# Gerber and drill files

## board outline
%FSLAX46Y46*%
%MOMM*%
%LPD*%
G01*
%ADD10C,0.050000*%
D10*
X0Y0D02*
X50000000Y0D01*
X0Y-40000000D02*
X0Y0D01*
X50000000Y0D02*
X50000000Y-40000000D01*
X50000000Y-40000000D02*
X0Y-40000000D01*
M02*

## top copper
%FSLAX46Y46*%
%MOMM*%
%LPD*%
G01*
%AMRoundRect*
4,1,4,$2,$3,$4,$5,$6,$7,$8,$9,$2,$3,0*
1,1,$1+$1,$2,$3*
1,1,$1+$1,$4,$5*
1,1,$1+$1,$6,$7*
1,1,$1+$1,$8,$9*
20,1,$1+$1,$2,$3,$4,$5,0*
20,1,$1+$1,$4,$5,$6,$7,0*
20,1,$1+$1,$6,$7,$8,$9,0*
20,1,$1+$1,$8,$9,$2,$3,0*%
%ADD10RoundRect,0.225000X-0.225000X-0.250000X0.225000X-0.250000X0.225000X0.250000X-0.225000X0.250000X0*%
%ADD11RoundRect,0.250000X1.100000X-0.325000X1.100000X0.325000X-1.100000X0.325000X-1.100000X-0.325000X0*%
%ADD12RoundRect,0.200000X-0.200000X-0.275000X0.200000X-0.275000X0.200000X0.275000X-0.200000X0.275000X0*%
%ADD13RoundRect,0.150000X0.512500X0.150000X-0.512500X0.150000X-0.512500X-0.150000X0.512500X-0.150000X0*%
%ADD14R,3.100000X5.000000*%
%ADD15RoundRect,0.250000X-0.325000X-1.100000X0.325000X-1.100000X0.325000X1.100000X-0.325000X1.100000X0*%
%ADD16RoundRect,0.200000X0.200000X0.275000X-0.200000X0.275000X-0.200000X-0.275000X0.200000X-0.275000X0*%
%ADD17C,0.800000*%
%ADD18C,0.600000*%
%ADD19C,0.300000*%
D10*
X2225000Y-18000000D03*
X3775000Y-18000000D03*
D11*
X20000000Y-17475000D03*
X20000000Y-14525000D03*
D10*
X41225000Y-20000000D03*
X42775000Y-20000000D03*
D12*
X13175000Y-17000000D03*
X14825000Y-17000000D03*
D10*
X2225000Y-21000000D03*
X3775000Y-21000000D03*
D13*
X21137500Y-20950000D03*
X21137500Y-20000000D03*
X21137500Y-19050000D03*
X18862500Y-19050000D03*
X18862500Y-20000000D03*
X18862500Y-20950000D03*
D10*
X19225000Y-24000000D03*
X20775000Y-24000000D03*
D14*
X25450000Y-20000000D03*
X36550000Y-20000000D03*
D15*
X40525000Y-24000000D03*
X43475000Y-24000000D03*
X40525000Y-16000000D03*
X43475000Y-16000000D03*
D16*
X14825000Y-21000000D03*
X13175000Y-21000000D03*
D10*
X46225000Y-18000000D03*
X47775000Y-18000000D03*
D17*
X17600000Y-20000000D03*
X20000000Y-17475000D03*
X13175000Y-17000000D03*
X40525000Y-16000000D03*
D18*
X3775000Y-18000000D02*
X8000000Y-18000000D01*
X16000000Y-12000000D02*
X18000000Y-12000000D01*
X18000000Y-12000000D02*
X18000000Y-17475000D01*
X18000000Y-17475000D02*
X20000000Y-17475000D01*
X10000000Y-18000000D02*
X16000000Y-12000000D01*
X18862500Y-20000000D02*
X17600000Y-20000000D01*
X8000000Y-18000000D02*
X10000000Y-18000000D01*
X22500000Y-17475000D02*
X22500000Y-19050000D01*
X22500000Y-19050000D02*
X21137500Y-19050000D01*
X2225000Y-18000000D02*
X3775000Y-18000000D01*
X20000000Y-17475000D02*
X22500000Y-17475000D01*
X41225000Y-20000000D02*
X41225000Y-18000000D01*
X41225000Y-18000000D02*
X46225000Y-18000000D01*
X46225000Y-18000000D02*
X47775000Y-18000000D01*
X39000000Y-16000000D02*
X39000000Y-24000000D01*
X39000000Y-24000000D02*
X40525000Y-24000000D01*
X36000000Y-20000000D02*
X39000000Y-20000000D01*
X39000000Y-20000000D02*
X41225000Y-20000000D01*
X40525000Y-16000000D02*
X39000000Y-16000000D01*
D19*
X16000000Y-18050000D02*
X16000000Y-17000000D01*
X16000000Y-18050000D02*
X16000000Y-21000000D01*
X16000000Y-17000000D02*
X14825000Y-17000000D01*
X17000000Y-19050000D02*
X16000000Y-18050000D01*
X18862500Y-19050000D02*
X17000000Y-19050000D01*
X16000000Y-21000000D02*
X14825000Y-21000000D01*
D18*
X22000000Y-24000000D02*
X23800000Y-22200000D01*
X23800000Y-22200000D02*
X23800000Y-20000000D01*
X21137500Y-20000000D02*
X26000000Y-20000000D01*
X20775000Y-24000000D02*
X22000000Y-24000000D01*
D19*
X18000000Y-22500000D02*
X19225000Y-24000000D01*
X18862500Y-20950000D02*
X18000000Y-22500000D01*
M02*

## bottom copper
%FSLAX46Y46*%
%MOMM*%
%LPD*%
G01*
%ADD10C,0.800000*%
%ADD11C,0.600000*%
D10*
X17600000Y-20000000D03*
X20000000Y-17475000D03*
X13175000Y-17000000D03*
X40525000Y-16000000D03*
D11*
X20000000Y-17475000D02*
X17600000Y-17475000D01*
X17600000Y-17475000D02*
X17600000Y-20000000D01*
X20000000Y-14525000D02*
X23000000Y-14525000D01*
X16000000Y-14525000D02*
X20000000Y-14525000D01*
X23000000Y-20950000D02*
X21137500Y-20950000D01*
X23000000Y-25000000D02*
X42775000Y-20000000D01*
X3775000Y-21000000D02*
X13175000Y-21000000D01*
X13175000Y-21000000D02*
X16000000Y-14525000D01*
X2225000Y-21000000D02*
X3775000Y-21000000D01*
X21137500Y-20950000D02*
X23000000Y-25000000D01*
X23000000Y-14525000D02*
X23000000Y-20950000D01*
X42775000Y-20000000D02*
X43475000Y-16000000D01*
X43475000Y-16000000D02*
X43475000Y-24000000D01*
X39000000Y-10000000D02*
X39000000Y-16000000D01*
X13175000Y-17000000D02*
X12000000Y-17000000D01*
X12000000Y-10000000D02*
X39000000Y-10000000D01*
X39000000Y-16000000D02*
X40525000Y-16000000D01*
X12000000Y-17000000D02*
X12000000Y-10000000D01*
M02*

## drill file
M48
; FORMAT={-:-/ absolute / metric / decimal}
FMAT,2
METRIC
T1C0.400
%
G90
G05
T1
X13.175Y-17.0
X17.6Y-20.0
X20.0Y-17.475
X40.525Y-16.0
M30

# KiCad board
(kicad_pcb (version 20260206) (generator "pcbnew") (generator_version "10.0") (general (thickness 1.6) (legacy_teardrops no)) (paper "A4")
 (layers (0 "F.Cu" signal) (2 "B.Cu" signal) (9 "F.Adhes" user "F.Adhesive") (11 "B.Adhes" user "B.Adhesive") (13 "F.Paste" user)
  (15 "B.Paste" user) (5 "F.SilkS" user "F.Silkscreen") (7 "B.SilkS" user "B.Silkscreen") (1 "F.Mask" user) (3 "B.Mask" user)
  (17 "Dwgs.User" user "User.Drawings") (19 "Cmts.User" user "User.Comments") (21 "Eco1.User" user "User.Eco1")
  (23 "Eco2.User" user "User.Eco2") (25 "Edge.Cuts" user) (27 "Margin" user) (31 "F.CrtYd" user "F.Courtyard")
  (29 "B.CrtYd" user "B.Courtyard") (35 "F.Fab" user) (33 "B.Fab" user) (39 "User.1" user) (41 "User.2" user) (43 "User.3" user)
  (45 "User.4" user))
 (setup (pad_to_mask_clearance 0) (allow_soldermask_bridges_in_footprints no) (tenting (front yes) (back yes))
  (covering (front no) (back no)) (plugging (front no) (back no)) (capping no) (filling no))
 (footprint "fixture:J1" (layer "F.Cu") (at 3 18)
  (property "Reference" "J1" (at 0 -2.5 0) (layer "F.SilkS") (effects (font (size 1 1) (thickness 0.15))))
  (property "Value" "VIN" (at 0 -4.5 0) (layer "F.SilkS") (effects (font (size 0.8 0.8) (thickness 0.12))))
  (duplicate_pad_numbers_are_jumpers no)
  (pad "1" smd roundrect (at -0.775 0) (size 0.9 0.95) (layers "F.Cu" "F.Mask" "F.Paste") (roundrect_rratio 0.25) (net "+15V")
   (thermal_bridge_angle 45))
  (pad "2" smd roundrect (at 0.775 0) (size 0.9 0.95) (layers "F.Cu" "F.Mask" "F.Paste") (roundrect_rratio 0.25) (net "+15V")
   (thermal_bridge_angle 45)))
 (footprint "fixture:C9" (layer "F.Cu") (at 20 16 90)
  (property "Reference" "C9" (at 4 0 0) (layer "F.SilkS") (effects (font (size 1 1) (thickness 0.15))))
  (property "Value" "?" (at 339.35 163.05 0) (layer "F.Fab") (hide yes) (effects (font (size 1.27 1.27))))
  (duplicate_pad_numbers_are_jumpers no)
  (pad "1" smd roundrect (at -1.475 0 90) (size 1.15 2.7) (layers "F.Cu" "F.Mask" "F.Paste") (roundrect_rratio 0.217391) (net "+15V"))
  (pad "2" smd roundrect (at 1.475 0 90) (size 1.15 2.7) (layers "F.Cu" "F.Mask" "F.Paste") (roundrect_rratio 0.217391) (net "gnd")))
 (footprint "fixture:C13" (layer "F.Cu") (at 42 20)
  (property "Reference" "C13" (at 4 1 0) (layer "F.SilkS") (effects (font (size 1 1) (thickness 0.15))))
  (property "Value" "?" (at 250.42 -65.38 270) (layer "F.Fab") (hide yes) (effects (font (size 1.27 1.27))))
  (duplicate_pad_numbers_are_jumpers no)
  (pad "1" smd roundrect (at -0.775 0) (size 0.9 0.95) (layers "F.Cu" "F.Mask" "F.Paste") (roundrect_rratio 0.25) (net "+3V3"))
  (pad "2" smd roundrect (at 0.775 0) (size 0.9 0.95) (layers "F.Cu" "F.Mask" "F.Paste") (roundrect_rratio 0.25) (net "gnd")))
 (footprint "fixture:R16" (layer "F.Cu") (at 14 17)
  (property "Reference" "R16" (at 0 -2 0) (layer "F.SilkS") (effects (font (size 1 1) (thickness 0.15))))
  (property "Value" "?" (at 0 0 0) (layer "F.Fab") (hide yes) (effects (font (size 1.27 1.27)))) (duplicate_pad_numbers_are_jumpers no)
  (pad "1" smd roundrect (at -0.825 0) (size 0.8 0.95) (layers "F.Cu" "F.Mask" "F.Paste") (roundrect_rratio 0.25) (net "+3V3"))
  (pad "2" smd roundrect (at 0.825 0) (size 0.8 0.95) (layers "F.Cu" "F.Mask" "F.Paste") (roundrect_rratio 0.25) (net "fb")))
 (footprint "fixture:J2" (layer "F.Cu") (at 3 21)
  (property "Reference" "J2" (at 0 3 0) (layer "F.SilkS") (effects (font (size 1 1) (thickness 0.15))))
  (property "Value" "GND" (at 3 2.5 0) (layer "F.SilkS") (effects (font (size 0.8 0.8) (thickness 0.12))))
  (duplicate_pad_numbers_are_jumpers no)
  (pad "1" smd roundrect (at -0.775 0) (size 0.9 0.95) (layers "F.Cu" "F.Mask" "F.Paste") (roundrect_rratio 0.25) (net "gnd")
   (thermal_bridge_angle 45))
  (pad "2" smd roundrect (at 0.775 0) (size 0.9 0.95) (layers "F.Cu" "F.Mask" "F.Paste") (roundrect_rratio 0.25) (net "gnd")
   (thermal_bridge_angle 45)))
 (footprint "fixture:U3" (layer "F.Cu") (at 20 20 180)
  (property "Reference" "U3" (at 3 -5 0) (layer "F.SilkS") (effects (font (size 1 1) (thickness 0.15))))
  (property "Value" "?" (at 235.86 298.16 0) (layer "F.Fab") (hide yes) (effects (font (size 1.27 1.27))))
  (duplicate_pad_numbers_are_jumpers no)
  (pad "1" smd roundrect (at -1.1375 -0.95 180) (size 1.325 0.6) (layers "F.Cu" "F.Mask" "F.Paste") (roundrect_rratio 0.25) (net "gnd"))
  (pad "2" smd roundrect (at -1.1375 0 180) (size 1.325 0.6) (layers "F.Cu" "F.Mask" "F.Paste") (roundrect_rratio 0.25) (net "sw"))
  (pad "3" smd roundrect (at -1.1375 0.95 180) (size 1.325 0.6) (layers "F.Cu" "F.Mask" "F.Paste") (roundrect_rratio 0.25) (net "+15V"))
  (pad "4" smd roundrect (at 1.1375 0.95 180) (size 1.325 0.6) (layers "F.Cu" "F.Mask" "F.Paste") (roundrect_rratio 0.25) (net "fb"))
  (pad "5" smd roundrect (at 1.1375 0 180) (size 1.325 0.6) (layers "F.Cu" "F.Mask" "F.Paste") (roundrect_rratio 0.25) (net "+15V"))
  (pad "6" smd roundrect (at 1.1375 -0.95 180) (size 1.325 0.6) (layers "F.Cu" "F.Mask" "F.Paste") (roundrect_rratio 0.25) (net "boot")))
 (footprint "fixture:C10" (layer "F.Cu") (at 20 24)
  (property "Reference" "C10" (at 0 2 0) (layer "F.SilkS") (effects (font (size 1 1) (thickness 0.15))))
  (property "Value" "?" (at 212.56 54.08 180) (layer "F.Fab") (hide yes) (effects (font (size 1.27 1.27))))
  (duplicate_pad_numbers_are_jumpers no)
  (pad "1" smd roundrect (at -0.775 0) (size 0.9 0.95) (layers "F.Cu" "F.Mask" "F.Paste") (roundrect_rratio 0.25) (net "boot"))
  (pad "2" smd roundrect (at 0.775 0) (size 0.9 0.95) (layers "F.Cu" "F.Mask" "F.Paste") (roundrect_rratio 0.25) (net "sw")))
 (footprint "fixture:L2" (layer "F.Cu") (at 31 20)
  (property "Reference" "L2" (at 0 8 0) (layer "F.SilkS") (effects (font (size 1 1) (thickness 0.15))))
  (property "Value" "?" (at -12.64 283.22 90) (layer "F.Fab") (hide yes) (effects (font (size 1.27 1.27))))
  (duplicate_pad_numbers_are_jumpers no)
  (pad "1" smd rect (at -5.55 0) (size 3.1 5) (layers "F.Cu" "F.Mask" "F.Paste") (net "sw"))
  (pad "2" smd rect (at 5.55 0) (size 3.1 5) (layers "F.Cu" "F.Mask" "F.Paste") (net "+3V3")))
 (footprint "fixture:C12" (layer "F.Cu") (at 42 24)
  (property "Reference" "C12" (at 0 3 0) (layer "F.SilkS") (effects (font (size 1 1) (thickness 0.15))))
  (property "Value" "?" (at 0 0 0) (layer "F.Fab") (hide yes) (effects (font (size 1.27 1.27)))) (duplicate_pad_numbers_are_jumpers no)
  (pad "1" smd roundrect (at -1.475 0) (size 1.15 2.7) (layers "F.Cu" "F.Mask" "F.Paste") (roundrect_rratio 0.217391) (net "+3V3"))
  (pad "2" smd roundrect (at 1.475 0) (size 1.15 2.7) (layers "F.Cu" "F.Mask" "F.Paste") (roundrect_rratio 0.217391) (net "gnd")))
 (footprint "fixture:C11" (layer "F.Cu") (at 42 16)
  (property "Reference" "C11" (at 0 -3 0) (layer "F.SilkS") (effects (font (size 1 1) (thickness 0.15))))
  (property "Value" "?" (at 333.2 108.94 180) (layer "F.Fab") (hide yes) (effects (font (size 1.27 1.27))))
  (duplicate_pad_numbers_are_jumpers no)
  (pad "1" smd roundrect (at -1.475 0) (size 1.15 2.7) (layers "F.Cu" "F.Mask" "F.Paste") (roundrect_rratio 0.217391) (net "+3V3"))
  (pad "2" smd roundrect (at 1.475 0) (size 1.15 2.7) (layers "F.Cu" "F.Mask" "F.Paste") (roundrect_rratio 0.217391) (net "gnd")))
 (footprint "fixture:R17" (layer "F.Cu") (at 14 21 180)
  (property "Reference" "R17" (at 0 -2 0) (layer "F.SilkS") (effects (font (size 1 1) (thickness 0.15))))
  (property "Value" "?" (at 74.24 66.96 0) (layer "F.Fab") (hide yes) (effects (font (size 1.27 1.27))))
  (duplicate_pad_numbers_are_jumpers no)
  (pad "1" smd roundrect (at -0.825 0 180) (size 0.8 0.95) (layers "F.Cu" "F.Mask" "F.Paste") (roundrect_rratio 0.25) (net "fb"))
  (pad "2" smd roundrect (at 0.825 0 180) (size 0.8 0.95) (layers "F.Cu" "F.Mask" "F.Paste") (roundrect_rratio 0.25) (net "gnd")))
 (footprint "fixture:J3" (layer "F.Cu") (at 47 18)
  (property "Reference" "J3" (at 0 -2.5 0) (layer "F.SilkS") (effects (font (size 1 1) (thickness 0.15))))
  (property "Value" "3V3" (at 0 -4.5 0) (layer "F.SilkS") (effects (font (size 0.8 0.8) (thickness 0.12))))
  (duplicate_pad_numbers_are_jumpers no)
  (pad "1" smd roundrect (at -0.775 0) (size 0.9 0.95) (layers "F.Cu" "F.Mask" "F.Paste") (roundrect_rratio 0.25) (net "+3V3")
   (thermal_bridge_angle 45))
  (pad "2" smd roundrect (at 0.775 0) (size 0.9 0.95) (layers "F.Cu" "F.Mask" "F.Paste") (roundrect_rratio 0.25) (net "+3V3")
   (thermal_bridge_angle 45)))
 (gr_line (start 0 0) (end 50 0) (stroke (width 0.05) (type default)) (layer "Edge.Cuts"))
 (gr_line (start 0 40) (end 0 0) (stroke (width 0.05) (type default)) (layer "Edge.Cuts"))
 (gr_line (start 50 0) (end 50 40) (stroke (width 0.05) (type default)) (layer "Edge.Cuts"))
 (gr_line (start 50 40) (end 0 40) (stroke (width 0.05) (type default)) (layer "Edge.Cuts"))
 (segment (start 3.775 18) (end 8 18) (width 0.6) (layer "F.Cu") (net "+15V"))
 (segment (start 16 12) (end 18 12) (width 0.6) (layer "F.Cu") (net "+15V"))
 (segment (start 18 12) (end 18 17.475) (width 0.6) (layer "F.Cu") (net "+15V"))
 (segment (start 18 17.475) (end 20 17.475) (width 0.6) (layer "F.Cu") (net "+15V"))
 (segment (start 10 18) (end 16 12) (width 0.6) (layer "F.Cu") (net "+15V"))
 (segment (start 18.8625 20) (end 17.6 20) (width 0.6) (layer "F.Cu") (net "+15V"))
 (segment (start 8 18) (end 10 18) (width 0.6) (layer "F.Cu") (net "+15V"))
 (segment (start 22.5 17.475) (end 22.5 19.05) (width 0.6) (layer "F.Cu") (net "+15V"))
 (segment (start 22.5 19.05) (end 21.1375 19.05) (width 0.6) (layer "F.Cu") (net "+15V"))
 (segment (start 2.225 18) (end 3.775 18) (width 0.6) (layer "F.Cu") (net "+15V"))
 (segment (start 20 17.475) (end 22.5 17.475) (width 0.6) (layer "F.Cu") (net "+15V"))
 (via (at 17.6 20) (size 0.8) (drill 0.4) (layers "F.Cu" "B.Cu") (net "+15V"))
 (via (at 20 17.475) (size 0.8) (drill 0.4) (layers "F.Cu" "B.Cu") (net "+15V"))
 (segment (start 20 17.475) (end 17.6 17.475) (width 0.6) (layer "B.Cu") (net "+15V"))
 (segment (start 17.6 17.475) (end 17.6 20) (width 0.6) (layer "B.Cu") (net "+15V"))
 (segment (start 20 14.525) (end 23 14.525) (width 0.6) (layer "B.Cu") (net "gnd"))
 (segment (start 16 14.525) (end 20 14.525) (width 0.6) (layer "B.Cu") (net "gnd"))
 (segment (start 23 20.95) (end 21.1375 20.95) (width 0.6) (layer "B.Cu") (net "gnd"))
 (segment (start 23 25) (end 42.775 20) (width 0.6) (layer "B.Cu") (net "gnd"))
 (segment (start 3.775 21) (end 13.175 21) (width 0.6) (layer "B.Cu") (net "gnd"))
 (segment (start 13.175 21) (end 16 14.525) (width 0.6) (layer "B.Cu") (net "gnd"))
 (segment (start 2.225 21) (end 3.775 21) (width 0.6) (layer "B.Cu") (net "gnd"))
 (segment (start 21.1375 20.95) (end 23 25) (width 0.6) (layer "B.Cu") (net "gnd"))
 (segment (start 23 14.525) (end 23 20.95) (width 0.6) (layer "B.Cu") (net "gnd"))
 (segment (start 42.775 20) (end 43.475 16) (width 0.6) (layer "B.Cu") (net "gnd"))
 (segment (start 43.475 16) (end 43.475 24) (width 0.6) (layer "B.Cu") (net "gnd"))
 (segment (start 41.225 20) (end 41.225 18) (width 0.6) (layer "F.Cu") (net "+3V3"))
 (segment (start 41.225 18) (end 46.225 18) (width 0.6) (layer "F.Cu") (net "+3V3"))
 (segment (start 46.225 18) (end 47.775 18) (width 0.6) (layer "F.Cu") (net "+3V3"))
 (segment (start 39 16) (end 39 24) (width 0.6) (layer "F.Cu") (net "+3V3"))
 (segment (start 39 24) (end 40.525 24) (width 0.6) (layer "F.Cu") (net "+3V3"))
 (segment (start 36 20) (end 39 20) (width 0.6) (layer "F.Cu") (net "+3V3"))
 (segment (start 39 20) (end 41.225 20) (width 0.6) (layer "F.Cu") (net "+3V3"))
 (segment (start 40.525 16) (end 39 16) (width 0.6) (layer "F.Cu") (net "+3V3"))
 (via (at 13.175 17) (size 0.8) (drill 0.4) (layers "F.Cu" "B.Cu") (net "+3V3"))
 (via (at 40.525 16) (size 0.8) (drill 0.4) (layers "F.Cu" "B.Cu") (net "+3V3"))
 (segment (start 39 10) (end 39 16) (width 0.6) (layer "B.Cu") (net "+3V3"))
 (segment (start 13.175 17) (end 12 17) (width 0.6) (layer "B.Cu") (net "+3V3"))
 (segment (start 12 10) (end 39 10) (width 0.6) (layer "B.Cu") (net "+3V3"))
 (segment (start 39 16) (end 40.525 16) (width 0.6) (layer "B.Cu") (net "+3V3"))
 (segment (start 12 17) (end 12 10) (width 0.6) (layer "B.Cu") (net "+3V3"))
 (segment (start 16 18.05) (end 16 17) (width 0.3) (layer "F.Cu") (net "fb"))
 (segment (start 16 18.05) (end 16 21) (width 0.3) (layer "F.Cu") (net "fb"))
 (segment (start 16 17) (end 14.825 17) (width 0.3) (layer "F.Cu") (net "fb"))
 (segment (start 17 19.05) (end 16 18.05) (width 0.3) (layer "F.Cu") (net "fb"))
 (segment (start 18.8625 19.05) (end 17 19.05) (width 0.3) (layer "F.Cu") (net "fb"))
 (segment (start 16 21) (end 14.825 21) (width 0.3) (layer "F.Cu") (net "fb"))
 (segment (start 22 24) (end 23.8 22.2) (width 0.6) (layer "F.Cu") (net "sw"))
 (segment (start 23.8 22.2) (end 23.8 20) (width 0.6) (layer "F.Cu") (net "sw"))
 (segment (start 21.1375 20) (end 26 20) (width 0.6) (layer "F.Cu") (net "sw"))
 (segment (start 20.775 24) (end 22 24) (width 0.6) (layer "F.Cu") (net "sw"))
 (segment (start 18 22.5) (end 19.225 24) (width 0.3) (layer "F.Cu") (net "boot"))
 (segment (start 18.8625 20.95) (end 18 22.5) (width 0.3) (layer "F.Cu") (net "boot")))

